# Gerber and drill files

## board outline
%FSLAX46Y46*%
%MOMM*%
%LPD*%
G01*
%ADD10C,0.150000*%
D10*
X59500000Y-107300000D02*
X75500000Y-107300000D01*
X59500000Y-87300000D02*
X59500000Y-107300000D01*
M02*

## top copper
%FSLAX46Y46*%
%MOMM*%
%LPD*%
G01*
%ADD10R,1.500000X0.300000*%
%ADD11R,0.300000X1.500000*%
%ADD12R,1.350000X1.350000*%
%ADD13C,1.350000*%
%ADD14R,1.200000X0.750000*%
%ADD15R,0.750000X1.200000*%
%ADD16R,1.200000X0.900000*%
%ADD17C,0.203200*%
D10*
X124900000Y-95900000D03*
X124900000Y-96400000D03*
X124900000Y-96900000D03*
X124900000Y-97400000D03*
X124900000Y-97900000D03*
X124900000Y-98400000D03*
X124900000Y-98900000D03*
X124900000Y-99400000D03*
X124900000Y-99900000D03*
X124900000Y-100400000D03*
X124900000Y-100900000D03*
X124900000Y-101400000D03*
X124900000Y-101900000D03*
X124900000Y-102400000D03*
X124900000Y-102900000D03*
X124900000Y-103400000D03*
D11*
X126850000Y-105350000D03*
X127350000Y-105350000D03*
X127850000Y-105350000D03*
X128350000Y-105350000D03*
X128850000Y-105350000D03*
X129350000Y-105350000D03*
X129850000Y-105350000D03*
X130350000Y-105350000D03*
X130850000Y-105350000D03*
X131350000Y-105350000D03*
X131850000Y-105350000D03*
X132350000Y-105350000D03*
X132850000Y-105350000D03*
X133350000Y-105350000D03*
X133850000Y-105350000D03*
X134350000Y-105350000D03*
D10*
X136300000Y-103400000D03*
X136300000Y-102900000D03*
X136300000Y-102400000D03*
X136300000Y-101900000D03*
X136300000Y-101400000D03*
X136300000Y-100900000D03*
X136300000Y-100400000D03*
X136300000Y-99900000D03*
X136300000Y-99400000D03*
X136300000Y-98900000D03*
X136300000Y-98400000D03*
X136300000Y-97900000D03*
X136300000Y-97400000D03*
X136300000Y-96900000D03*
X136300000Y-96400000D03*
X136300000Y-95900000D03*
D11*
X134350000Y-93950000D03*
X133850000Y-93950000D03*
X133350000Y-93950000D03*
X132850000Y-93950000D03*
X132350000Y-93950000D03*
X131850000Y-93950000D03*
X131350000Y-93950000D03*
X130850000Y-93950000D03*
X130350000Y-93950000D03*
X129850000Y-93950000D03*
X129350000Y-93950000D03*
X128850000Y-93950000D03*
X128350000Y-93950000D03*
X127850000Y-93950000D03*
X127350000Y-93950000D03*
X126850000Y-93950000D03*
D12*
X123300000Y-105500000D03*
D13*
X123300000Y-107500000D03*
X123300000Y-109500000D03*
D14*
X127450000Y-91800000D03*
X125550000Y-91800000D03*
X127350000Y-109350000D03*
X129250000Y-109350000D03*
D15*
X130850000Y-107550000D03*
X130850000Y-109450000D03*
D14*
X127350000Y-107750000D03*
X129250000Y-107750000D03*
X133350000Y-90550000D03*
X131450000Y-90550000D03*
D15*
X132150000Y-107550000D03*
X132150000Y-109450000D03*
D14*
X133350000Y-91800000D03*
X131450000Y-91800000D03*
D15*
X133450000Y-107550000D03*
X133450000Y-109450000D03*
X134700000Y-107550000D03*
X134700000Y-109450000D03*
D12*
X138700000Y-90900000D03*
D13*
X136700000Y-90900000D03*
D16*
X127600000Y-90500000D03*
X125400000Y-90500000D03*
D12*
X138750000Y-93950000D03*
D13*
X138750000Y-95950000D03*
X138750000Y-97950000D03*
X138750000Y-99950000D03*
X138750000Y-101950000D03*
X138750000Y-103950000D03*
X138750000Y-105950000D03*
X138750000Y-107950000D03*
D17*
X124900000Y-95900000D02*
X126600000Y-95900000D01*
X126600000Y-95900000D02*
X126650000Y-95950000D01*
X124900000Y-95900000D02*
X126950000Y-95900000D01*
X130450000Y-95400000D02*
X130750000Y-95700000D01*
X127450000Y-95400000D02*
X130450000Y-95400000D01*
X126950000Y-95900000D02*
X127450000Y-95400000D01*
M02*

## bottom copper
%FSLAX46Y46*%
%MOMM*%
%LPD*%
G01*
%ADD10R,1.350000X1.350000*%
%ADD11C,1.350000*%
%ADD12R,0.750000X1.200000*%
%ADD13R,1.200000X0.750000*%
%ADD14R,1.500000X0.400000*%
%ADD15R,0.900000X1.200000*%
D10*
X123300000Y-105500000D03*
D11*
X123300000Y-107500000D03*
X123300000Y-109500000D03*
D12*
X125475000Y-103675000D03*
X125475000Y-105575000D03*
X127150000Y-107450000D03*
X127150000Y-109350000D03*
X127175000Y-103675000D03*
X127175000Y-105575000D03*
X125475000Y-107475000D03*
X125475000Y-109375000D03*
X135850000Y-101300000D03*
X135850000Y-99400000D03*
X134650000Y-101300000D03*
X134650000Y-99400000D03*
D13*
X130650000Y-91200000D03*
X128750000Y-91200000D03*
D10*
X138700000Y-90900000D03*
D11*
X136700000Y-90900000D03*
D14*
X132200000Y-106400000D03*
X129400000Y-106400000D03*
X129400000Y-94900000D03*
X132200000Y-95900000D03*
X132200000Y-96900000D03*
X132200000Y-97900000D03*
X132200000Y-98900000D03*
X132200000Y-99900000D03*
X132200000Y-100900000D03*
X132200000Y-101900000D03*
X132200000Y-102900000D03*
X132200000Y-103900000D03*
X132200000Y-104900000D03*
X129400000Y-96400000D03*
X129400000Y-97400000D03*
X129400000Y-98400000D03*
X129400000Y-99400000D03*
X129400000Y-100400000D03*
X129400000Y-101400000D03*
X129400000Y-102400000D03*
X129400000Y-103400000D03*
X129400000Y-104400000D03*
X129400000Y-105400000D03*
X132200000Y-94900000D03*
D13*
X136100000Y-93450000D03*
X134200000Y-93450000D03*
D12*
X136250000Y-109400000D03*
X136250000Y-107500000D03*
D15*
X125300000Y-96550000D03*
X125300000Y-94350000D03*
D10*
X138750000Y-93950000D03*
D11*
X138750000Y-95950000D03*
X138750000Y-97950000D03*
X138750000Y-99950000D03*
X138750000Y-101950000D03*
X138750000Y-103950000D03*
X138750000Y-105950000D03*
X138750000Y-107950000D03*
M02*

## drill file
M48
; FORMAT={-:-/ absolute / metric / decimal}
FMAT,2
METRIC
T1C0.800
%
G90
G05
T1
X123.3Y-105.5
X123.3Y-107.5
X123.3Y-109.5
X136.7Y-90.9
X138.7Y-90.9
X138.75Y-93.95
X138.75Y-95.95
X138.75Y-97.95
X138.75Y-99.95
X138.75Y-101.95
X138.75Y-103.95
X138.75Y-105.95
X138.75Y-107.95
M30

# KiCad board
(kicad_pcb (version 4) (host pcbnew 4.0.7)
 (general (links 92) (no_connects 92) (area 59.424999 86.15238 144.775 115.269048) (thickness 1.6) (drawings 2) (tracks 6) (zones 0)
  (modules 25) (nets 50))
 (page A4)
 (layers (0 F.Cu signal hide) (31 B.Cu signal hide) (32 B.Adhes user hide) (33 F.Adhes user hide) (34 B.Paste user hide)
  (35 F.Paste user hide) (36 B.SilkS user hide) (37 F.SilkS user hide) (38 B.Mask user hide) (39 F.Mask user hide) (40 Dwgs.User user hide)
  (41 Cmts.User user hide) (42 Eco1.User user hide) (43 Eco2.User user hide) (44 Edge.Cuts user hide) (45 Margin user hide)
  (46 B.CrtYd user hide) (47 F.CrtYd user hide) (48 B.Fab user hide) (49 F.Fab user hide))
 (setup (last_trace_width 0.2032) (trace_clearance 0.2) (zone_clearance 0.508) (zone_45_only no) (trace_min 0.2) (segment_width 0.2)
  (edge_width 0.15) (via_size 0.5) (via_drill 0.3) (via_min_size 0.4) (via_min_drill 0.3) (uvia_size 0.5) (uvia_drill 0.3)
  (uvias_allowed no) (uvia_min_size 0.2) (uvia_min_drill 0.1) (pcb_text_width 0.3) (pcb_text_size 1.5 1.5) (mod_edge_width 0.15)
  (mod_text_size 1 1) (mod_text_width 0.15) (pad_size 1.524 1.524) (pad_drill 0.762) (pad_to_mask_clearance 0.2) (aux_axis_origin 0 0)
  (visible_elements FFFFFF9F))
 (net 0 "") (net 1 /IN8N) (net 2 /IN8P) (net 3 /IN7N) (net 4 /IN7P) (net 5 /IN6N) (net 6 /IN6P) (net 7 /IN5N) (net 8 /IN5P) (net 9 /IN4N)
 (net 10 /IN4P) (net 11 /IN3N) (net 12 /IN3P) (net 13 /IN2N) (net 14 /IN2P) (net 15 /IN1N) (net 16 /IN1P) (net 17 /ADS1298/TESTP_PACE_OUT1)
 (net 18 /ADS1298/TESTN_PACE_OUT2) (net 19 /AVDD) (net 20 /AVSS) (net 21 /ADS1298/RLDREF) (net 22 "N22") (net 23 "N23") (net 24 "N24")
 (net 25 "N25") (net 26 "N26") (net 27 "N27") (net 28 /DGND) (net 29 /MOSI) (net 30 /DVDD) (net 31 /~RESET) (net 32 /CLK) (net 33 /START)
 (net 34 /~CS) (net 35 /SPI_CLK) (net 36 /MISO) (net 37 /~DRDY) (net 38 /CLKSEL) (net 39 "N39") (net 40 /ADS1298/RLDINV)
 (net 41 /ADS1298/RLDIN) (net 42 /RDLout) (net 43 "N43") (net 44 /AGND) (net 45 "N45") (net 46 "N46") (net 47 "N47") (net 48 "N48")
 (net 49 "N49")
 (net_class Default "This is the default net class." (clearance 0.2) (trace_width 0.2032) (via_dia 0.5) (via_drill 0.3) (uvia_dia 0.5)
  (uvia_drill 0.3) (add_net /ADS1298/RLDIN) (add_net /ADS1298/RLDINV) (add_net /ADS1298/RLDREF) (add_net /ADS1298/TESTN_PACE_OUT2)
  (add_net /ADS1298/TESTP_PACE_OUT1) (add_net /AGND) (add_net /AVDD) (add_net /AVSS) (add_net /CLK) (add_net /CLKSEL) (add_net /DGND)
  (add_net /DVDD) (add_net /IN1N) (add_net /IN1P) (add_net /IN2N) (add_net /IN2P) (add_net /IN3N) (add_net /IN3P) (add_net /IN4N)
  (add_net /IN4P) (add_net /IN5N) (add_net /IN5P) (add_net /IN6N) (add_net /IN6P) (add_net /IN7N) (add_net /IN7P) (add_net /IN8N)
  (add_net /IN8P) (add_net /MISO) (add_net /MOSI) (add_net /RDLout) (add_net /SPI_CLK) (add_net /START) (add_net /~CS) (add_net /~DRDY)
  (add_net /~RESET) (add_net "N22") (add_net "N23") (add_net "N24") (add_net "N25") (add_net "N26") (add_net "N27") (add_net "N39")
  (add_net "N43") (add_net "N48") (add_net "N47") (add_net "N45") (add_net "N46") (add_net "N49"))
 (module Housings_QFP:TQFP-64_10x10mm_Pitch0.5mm (layer F.Cu) (at 130.6 99.65)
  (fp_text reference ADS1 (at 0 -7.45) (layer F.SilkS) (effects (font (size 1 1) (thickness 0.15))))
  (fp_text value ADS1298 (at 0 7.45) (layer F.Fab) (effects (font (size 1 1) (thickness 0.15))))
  (pad 1 smd rect (at -5.7 -3.75) (size 1.5 0.3) (layers F.Cu F.Paste F.Mask) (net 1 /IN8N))
  (pad 2 smd rect (at -5.7 -3.25) (size 1.5 0.3) (layers F.Cu F.Paste F.Mask) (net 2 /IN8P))
  (pad 3 smd rect (at -5.7 -2.75) (size 1.5 0.3) (layers F.Cu F.Paste F.Mask) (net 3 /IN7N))
  (pad 4 smd rect (at -5.7 -2.25) (size 1.5 0.3) (layers F.Cu F.Paste F.Mask) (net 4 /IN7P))
  (pad 5 smd rect (at -5.7 -1.75) (size 1.5 0.3) (layers F.Cu F.Paste F.Mask) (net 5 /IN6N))
  (pad 6 smd rect (at -5.7 -1.25) (size 1.5 0.3) (layers F.Cu F.Paste F.Mask) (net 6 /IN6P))
  (pad 7 smd rect (at -5.7 -0.75) (size 1.5 0.3) (layers F.Cu F.Paste F.Mask) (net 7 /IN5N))
  (pad 8 smd rect (at -5.7 -0.25) (size 1.5 0.3) (layers F.Cu F.Paste F.Mask) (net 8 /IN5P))
  (pad 9 smd rect (at -5.7 0.25) (size 1.5 0.3) (layers F.Cu F.Paste F.Mask) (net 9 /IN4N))
  (pad 10 smd rect (at -5.7 0.75) (size 1.5 0.3) (layers F.Cu F.Paste F.Mask) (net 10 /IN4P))
  (pad 11 smd rect (at -5.7 1.25) (size 1.5 0.3) (layers F.Cu F.Paste F.Mask) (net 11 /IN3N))
  (pad 12 smd rect (at -5.7 1.75) (size 1.5 0.3) (layers F.Cu F.Paste F.Mask) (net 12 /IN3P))
  (pad 13 smd rect (at -5.7 2.25) (size 1.5 0.3) (layers F.Cu F.Paste F.Mask) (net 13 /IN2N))
  (pad 14 smd rect (at -5.7 2.75) (size 1.5 0.3) (layers F.Cu F.Paste F.Mask) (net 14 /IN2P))
  (pad 15 smd rect (at -5.7 3.25) (size 1.5 0.3) (layers F.Cu F.Paste F.Mask) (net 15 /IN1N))
  (pad 16 smd rect (at -5.7 3.75) (size 1.5 0.3) (layers F.Cu F.Paste F.Mask) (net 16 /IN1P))
  (pad 17 smd rect (at -3.75 5.7 90) (size 1.5 0.3) (layers F.Cu F.Paste F.Mask) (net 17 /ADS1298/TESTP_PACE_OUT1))
  (pad 18 smd rect (at -3.25 5.7 90) (size 1.5 0.3) (layers F.Cu F.Paste F.Mask) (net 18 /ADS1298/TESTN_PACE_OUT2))
  (pad 19 smd rect (at -2.75 5.7 90) (size 1.5 0.3) (layers F.Cu F.Paste F.Mask) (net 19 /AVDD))
  (pad 20 smd rect (at -2.25 5.7 90) (size 1.5 0.3) (layers F.Cu F.Paste F.Mask) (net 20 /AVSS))
  (pad 21 smd rect (at -1.75 5.7 90) (size 1.5 0.3) (layers F.Cu F.Paste F.Mask) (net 19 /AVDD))
  (pad 22 smd rect (at -1.25 5.7 90) (size 1.5 0.3) (layers F.Cu F.Paste F.Mask) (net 19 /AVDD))
  (pad 23 smd rect (at -0.75 5.7 90) (size 1.5 0.3) (layers F.Cu F.Paste F.Mask) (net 20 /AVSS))
  (pad 24 smd rect (at -0.25 5.7 90) (size 1.5 0.3) (layers F.Cu F.Paste F.Mask) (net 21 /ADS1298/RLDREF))
  (pad 25 smd rect (at 0.25 5.7 90) (size 1.5 0.3) (layers F.Cu F.Paste F.Mask) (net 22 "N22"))
  (pad 26 smd rect (at 0.75 5.7 90) (size 1.5 0.3) (layers F.Cu F.Paste F.Mask) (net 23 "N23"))
  (pad 27 smd rect (at 1.25 5.7 90) (size 1.5 0.3) (layers F.Cu F.Paste F.Mask) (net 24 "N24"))
  (pad 28 smd rect (at 1.75 5.7 90) (size 1.5 0.3) (layers F.Cu F.Paste F.Mask) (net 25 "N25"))
  (pad 29 smd rect (at 2.25 5.7 90) (size 1.5 0.3) (layers F.Cu F.Paste F.Mask) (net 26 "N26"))
  (pad 30 smd rect (at 2.75 5.7 90) (size 1.5 0.3) (layers F.Cu F.Paste F.Mask) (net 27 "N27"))
  (pad 31 smd rect (at 3.25 5.7 90) (size 1.5 0.3) (layers F.Cu F.Paste F.Mask) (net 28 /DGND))
  (pad 32 smd rect (at 3.75 5.7 90) (size 1.5 0.3) (layers F.Cu F.Paste F.Mask) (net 20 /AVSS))
  (pad 33 smd rect (at 5.7 3.75) (size 1.5 0.3) (layers F.Cu F.Paste F.Mask) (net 28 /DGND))
  (pad 34 smd rect (at 5.7 3.25) (size 1.5 0.3) (layers F.Cu F.Paste F.Mask) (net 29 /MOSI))
  (pad 35 smd rect (at 5.7 2.75) (size 1.5 0.3) (layers F.Cu F.Paste F.Mask) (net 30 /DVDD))
  (pad 36 smd rect (at 5.7 2.25) (size 1.5 0.3) (layers F.Cu F.Paste F.Mask) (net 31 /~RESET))
  (pad 37 smd rect (at 5.7 1.75) (size 1.5 0.3) (layers F.Cu F.Paste F.Mask) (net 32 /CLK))
  (pad 38 smd rect (at 5.7 1.25) (size 1.5 0.3) (layers F.Cu F.Paste F.Mask) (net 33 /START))
  (pad 39 smd rect (at 5.7 0.75) (size 1.5 0.3) (layers F.Cu F.Paste F.Mask) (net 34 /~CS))
  (pad 40 smd rect (at 5.7 0.25) (size 1.5 0.3) (layers F.Cu F.Paste F.Mask) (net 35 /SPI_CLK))
  (pad 41 smd rect (at 5.7 -0.25) (size 1.5 0.3) (layers F.Cu F.Paste F.Mask) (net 28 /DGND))
  (pad 42 smd rect (at 5.7 -0.75) (size 1.5 0.3) (layers F.Cu F.Paste F.Mask) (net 28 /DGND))
  (pad 43 smd rect (at 5.7 -1.25) (size 1.5 0.3) (layers F.Cu F.Paste F.Mask) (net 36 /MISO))
  (pad 44 smd rect (at 5.7 -1.75) (size 1.5 0.3) (layers F.Cu F.Paste F.Mask) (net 28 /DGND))
  (pad 45 smd rect (at 5.7 -2.25) (size 1.5 0.3) (layers F.Cu F.Paste F.Mask) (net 28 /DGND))
  (pad 46 smd rect (at 5.7 -2.75) (size 1.5 0.3) (layers F.Cu F.Paste F.Mask) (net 28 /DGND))
  (pad 47 smd rect (at 5.7 -3.25) (size 1.5 0.3) (layers F.Cu F.Paste F.Mask) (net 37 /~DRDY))
  (pad 48 smd rect (at 5.7 -3.75) (size 1.5 0.3) (layers F.Cu F.Paste F.Mask) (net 30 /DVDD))
  (pad 49 smd rect (at 3.75 -5.7 90) (size 1.5 0.3) (layers F.Cu F.Paste F.Mask) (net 28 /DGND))
  (pad 50 smd rect (at 3.25 -5.7 90) (size 1.5 0.3) (layers F.Cu F.Paste F.Mask) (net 30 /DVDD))
  (pad 51 smd rect (at 2.75 -5.7 90) (size 1.5 0.3) (layers F.Cu F.Paste F.Mask) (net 28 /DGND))
  (pad 52 smd rect (at 2.25 -5.7 90) (size 1.5 0.3) (layers F.Cu F.Paste F.Mask) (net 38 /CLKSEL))
  (pad 53 smd rect (at 1.75 -5.7 90) (size 1.5 0.3) (layers F.Cu F.Paste F.Mask) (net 20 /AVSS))
  (pad 54 smd rect (at 1.25 -5.7 90) (size 1.5 0.3) (layers F.Cu F.Paste F.Mask) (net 19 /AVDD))
  (pad 55 smd rect (at 0.75 -5.7 90) (size 1.5 0.3) (layers F.Cu F.Paste F.Mask) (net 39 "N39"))
  (pad 56 smd rect (at 0.25 -5.7 90) (size 1.5 0.3) (layers F.Cu F.Paste F.Mask) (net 19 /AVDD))
  (pad 57 smd rect (at -0.25 -5.7 90) (size 1.5 0.3) (layers F.Cu F.Paste F.Mask) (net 20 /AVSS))
  (pad 58 smd rect (at -0.75 -5.7 90) (size 1.5 0.3) (layers F.Cu F.Paste F.Mask) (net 20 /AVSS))
  (pad 59 smd rect (at -1.25 -5.7 90) (size 1.5 0.3) (layers F.Cu F.Paste F.Mask) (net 19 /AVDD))
  (pad 60 smd rect (at -1.75 -5.7 90) (size 1.5 0.3) (layers F.Cu F.Paste F.Mask) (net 21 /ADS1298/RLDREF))
  (pad 61 smd rect (at -2.25 -5.7 90) (size 1.5 0.3) (layers F.Cu F.Paste F.Mask) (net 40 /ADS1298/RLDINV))
  (pad 62 smd rect (at -2.75 -5.7 90) (size 1.5 0.3) (layers F.Cu F.Paste F.Mask) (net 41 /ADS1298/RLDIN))
  (pad 63 smd rect (at -3.25 -5.7 90) (size 1.5 0.3) (layers F.Cu F.Paste F.Mask) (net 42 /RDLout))
  (pad 64 smd rect (at -3.75 -5.7 90) (size 1.5 0.3) (layers F.Cu F.Paste F.Mask) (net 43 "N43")))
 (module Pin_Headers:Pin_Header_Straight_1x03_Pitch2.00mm (layer F.Cu) (at 123.3 105.5)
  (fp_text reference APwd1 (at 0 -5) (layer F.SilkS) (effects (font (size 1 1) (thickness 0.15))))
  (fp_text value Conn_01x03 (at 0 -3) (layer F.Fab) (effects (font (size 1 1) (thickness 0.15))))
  (pad 1 thru_hole rect (at 0 0) (size 1.35 1.35) (drill 0.8) (layers *.Cu *.Mask) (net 19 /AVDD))
  (pad 2 thru_hole circle (at 0 2) (size 1.35 1.35) (drill 0.8) (layers *.Cu *.Mask) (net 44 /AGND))
  (pad 3 thru_hole circle (at 0 4) (size 1.35 1.35) (drill 0.8) (layers *.Cu *.Mask) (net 20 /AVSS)))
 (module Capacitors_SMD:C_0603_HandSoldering (layer F.Cu) (at 126.5 91.8 180)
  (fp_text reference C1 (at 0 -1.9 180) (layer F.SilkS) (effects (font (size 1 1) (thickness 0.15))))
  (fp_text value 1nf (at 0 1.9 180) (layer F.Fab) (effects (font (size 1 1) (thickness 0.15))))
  (pad 1 smd rect (at -0.95 0 180) (size 1.2 0.75) (layers F.Cu F.Paste F.Mask) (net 40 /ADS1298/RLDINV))
  (pad 2 smd rect (at 0.95 0 180) (size 1.2 0.75) (layers F.Cu F.Paste F.Mask) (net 42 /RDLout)))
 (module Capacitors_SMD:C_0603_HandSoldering (layer B.Cu) (at 125.475 104.625 270)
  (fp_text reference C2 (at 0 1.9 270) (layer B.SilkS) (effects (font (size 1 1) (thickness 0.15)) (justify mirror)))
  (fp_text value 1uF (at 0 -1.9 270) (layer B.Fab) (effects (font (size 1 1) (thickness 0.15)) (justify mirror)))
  (pad 1 smd rect (at -0.95 0 270) (size 1.2 0.75) (layers B.Cu B.Paste B.Mask) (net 19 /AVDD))
  (pad 2 smd rect (at 0.95 0 270) (size 1.2 0.75) (layers B.Cu B.Paste B.Mask) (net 44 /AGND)))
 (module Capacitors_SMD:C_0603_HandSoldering (layer B.Cu) (at 127.15 108.4 270)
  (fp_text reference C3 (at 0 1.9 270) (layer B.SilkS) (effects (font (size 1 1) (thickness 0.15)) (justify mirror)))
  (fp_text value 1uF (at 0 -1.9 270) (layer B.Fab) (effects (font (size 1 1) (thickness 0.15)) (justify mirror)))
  (pad 1 smd rect (at -0.95 0 270) (size 1.2 0.75) (layers B.Cu B.Paste B.Mask) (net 44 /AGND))
  (pad 2 smd rect (at 0.95 0 270) (size 1.2 0.75) (layers B.Cu B.Paste B.Mask) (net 20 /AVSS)))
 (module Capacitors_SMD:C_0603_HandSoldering (layer B.Cu) (at 127.175 104.625 270)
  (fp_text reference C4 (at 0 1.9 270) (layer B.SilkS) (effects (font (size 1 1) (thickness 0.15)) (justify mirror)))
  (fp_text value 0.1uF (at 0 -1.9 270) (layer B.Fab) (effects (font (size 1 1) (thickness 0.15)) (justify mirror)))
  (pad 1 smd rect (at -0.95 0 270) (size 1.2 0.75) (layers B.Cu B.Paste B.Mask) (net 19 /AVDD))
  (pad 2 smd rect (at 0.95 0 270) (size 1.2 0.75) (layers B.Cu B.Paste B.Mask) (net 44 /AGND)))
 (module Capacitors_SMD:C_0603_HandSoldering (layer B.Cu) (at 125.475 108.425 270)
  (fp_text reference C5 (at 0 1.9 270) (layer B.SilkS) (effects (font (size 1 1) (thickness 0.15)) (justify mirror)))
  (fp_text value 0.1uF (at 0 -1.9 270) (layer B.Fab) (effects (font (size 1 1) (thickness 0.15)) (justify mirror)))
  (pad 1 smd rect (at -0.95 0 270) (size 1.2 0.75) (layers B.Cu B.Paste B.Mask) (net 44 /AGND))
  (pad 2 smd rect (at 0.95 0 270) (size 1.2 0.75) (layers B.Cu B.Paste B.Mask) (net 20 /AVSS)))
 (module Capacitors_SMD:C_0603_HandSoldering (layer B.Cu) (at 135.85 100.35 90)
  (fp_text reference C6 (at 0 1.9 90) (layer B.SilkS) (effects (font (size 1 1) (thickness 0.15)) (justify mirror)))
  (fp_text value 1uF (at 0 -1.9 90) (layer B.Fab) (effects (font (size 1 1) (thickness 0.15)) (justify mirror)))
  (pad 1 smd rect (at -0.95 0 90) (size 1.2 0.75) (layers B.Cu B.Paste B.Mask) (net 30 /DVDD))
  (pad 2 smd rect (at 0.95 0 90) (size 1.2 0.75) (layers B.Cu B.Paste B.Mask) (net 28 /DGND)))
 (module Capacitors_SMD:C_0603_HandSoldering (layer B.Cu) (at 134.65 100.35 90)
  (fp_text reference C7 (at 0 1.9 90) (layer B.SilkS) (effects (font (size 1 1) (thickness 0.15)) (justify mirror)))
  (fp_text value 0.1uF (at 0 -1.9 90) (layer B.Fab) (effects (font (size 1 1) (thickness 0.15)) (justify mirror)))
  (pad 1 smd rect (at -0.95 0 90) (size 1.2 0.75) (layers B.Cu B.Paste B.Mask) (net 30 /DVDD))
  (pad 2 smd rect (at 0.95 0 90) (size 1.2 0.75) (layers B.Cu B.Paste B.Mask) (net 28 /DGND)))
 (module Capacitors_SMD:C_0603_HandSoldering (layer B.Cu) (at 129.7 91.2 180)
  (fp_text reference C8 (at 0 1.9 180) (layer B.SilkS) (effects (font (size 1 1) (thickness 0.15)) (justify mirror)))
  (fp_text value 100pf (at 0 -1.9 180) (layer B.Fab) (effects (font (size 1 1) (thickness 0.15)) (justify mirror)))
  (pad 1 smd rect (at -0.95 0 180) (size 1.2 0.75) (layers B.Cu B.Paste B.Mask) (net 20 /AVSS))
  (pad 2 smd rect (at 0.95 0 180) (size 1.2 0.75) (layers B.Cu B.Paste B.Mask) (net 43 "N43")))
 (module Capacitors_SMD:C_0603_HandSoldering (layer F.Cu) (at 128.3 109.35)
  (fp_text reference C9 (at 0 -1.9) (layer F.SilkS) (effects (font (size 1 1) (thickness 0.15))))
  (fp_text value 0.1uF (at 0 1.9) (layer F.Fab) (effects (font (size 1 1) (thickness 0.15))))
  (pad 1 smd rect (at -0.95 0) (size 1.2 0.75) (layers F.Cu F.Paste F.Mask) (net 21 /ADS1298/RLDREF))
  (pad 2 smd rect (at 0.95 0) (size 1.2 0.75) (layers F.Cu F.Paste F.Mask) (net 22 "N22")))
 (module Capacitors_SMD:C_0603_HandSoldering (layer F.Cu) (at 130.85 108.5 270)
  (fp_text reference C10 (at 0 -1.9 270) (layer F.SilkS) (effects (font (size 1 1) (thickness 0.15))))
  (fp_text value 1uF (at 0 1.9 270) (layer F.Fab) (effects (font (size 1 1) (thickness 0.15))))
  (pad 1 smd rect (at -0.95 0 270) (size 1.2 0.75) (layers F.Cu F.Paste F.Mask) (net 22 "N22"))
  (pad 2 smd rect (at 0.95 0 270) (size 1.2 0.75) (layers F.Cu F.Paste F.Mask) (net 20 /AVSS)))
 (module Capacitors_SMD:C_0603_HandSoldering (layer F.Cu) (at 128.3 107.75)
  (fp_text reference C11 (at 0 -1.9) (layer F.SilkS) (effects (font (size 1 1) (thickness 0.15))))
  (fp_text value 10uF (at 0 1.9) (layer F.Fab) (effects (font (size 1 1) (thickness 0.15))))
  (pad 1 smd rect (at -0.95 0) (size 1.2 0.75) (layers F.Cu F.Paste F.Mask) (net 21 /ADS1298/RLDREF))
  (pad 2 smd rect (at 0.95 0) (size 1.2 0.75) (layers F.Cu F.Paste F.Mask) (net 22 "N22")))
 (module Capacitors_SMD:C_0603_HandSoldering (layer F.Cu) (at 132.4 90.55 180)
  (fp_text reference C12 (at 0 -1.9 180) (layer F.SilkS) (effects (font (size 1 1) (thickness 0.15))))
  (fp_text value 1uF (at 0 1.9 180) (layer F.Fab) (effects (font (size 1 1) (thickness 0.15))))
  (pad 1 smd rect (at -0.95 0 180) (size 1.2 0.75) (layers F.Cu F.Paste F.Mask) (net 20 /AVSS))
  (pad 2 smd rect (at 0.95 0 180) (size 1.2 0.75) (layers F.Cu F.Paste F.Mask) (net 39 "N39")))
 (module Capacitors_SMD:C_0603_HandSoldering (layer F.Cu) (at 132.15 108.5 270)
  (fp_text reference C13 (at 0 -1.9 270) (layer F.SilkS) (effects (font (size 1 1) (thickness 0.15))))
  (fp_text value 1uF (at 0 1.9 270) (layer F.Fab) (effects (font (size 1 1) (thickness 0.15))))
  (pad 1 smd rect (at -0.95 0 270) (size 1.2 0.75) (layers F.Cu F.Paste F.Mask) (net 23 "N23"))
  (pad 2 smd rect (at 0.95 0 270) (size 1.2 0.75) (layers F.Cu F.Paste F.Mask) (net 20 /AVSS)))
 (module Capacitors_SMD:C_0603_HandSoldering (layer F.Cu) (at 132.4 91.8 180)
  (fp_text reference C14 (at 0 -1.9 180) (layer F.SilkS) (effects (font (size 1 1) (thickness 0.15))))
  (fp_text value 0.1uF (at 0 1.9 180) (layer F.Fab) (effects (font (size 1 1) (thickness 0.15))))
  (pad 1 smd rect (at -0.95 0 180) (size 1.2 0.75) (layers F.Cu F.Paste F.Mask) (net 20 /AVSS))
  (pad 2 smd rect (at 0.95 0 180) (size 1.2 0.75) (layers F.Cu F.Paste F.Mask) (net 39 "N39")))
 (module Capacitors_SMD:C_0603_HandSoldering (layer F.Cu) (at 133.45 108.5 270)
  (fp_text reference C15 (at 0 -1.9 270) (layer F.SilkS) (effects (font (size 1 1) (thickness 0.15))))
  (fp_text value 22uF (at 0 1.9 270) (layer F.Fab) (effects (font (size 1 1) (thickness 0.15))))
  (pad 1 smd rect (at -0.95 0 270) (size 1.2 0.75) (layers F.Cu F.Paste F.Mask) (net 25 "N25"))
  (pad 2 smd rect (at 0.95 0 270) (size 1.2 0.75) (layers F.Cu F.Paste F.Mask) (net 20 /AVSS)))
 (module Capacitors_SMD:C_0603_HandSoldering (layer F.Cu) (at 134.7 108.5 270)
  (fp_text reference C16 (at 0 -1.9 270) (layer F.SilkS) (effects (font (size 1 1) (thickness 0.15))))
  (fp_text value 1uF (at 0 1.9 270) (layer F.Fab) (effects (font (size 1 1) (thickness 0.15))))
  (pad 1 smd rect (at -0.95 0 270) (size 1.2 0.75) (layers F.Cu F.Paste F.Mask) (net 27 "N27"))
  (pad 2 smd rect (at 0.95 0 270) (size 1.2 0.75) (layers F.Cu F.Paste F.Mask) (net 20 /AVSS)))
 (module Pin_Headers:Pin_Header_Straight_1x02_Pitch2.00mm (layer F.Cu) (at 138.7 90.9 270)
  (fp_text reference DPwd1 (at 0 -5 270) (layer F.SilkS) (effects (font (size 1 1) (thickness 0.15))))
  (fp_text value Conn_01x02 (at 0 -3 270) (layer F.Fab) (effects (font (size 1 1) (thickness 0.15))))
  (pad 1 thru_hole rect (at 0 0 270) (size 1.35 1.35) (drill 0.8) (layers *.Cu *.Mask) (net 30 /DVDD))
  (pad 2 thru_hole circle (at 0 2 270) (size 1.35 1.35) (drill 0.8) (layers *.Cu *.Mask) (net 28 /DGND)))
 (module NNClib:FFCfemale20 (layer B.Cu) (at 132.95 95.9 270)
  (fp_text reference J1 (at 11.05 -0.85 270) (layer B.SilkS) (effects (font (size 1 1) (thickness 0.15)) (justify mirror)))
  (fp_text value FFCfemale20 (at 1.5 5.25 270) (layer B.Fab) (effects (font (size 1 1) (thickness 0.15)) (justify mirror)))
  (pad 42 smd rect (at 10.5 0.75 270) (size 0.4 1.5) (layers B.Cu B.Paste B.Mask) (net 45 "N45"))
  (pad 43 smd rect (at 10.5 3.55 270) (size 0.4 1.5) (layers B.Cu B.Paste B.Mask) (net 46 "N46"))
  (pad 41 smd rect (at -1 3.55 270) (size 0.4 1.5) (layers B.Cu B.Paste B.Mask) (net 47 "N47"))
  (pad 1 smd rect (at 0 0.75 90) (size 0.4 1.5) (layers B.Cu B.Paste B.Mask) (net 44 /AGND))
  (pad 3 smd rect (at 1 0.75 90) (size 0.4 1.5) (layers B.Cu B.Paste B.Mask) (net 1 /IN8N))
  (pad 5 smd rect (at 2 0.75 90) (size 0.4 1.5) (layers B.Cu B.Paste B.Mask) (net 3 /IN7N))
  (pad 7 smd rect (at 3 0.75 90) (size 0.4 1.5) (layers B.Cu B.Paste B.Mask) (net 5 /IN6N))
  (pad 9 smd rect (at 4 0.75 90) (size 0.4 1.5) (layers B.Cu B.Paste B.Mask) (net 7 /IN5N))
  (pad 11 smd rect (at 5 0.75 90) (size 0.4 1.5) (layers B.Cu B.Paste B.Mask) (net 9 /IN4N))
  (pad 13 smd rect (at 6 0.75 90) (size 0.4 1.5) (layers B.Cu B.Paste B.Mask) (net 11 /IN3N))
  (pad 15 smd rect (at 7 0.75 90) (size 0.4 1.5) (layers B.Cu B.Paste B.Mask) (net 13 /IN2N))
  (pad 17 smd rect (at 8 0.75 90) (size 0.4 1.5) (layers B.Cu B.Paste B.Mask) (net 15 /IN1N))
  (pad 19 smd rect (at 9 0.75 90) (size 0.4 1.5) (layers B.Cu B.Paste B.Mask) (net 42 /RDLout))
  (pad 2 smd rect (at 0.5 3.55 90) (size 0.4 1.5) (layers B.Cu B.Paste B.Mask) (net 42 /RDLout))
  (pad 4 smd rect (at 1.5 3.55 90) (size 0.4 1.5) (layers B.Cu B.Paste B.Mask) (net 2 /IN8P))
  (pad 6 smd rect (at 2.5 3.55 90) (size 0.4 1.5) (layers B.Cu B.Paste B.Mask) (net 4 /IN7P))
  (pad 8 smd rect (at 3.5 3.55 90) (size 0.4 1.5) (layers B.Cu B.Paste B.Mask) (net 6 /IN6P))
  (pad 10 smd rect (at 4.5 3.55 90) (size 0.4 1.5) (layers B.Cu B.Paste B.Mask) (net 8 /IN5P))
  (pad 12 smd rect (at 5.5 3.55 90) (size 0.4 1.5) (layers B.Cu B.Paste B.Mask) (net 10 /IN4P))
  (pad 14 smd rect (at 6.5 3.55 90) (size 0.4 1.5) (layers B.Cu B.Paste B.Mask) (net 12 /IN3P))
  (pad 16 smd rect (at 7.5 3.55 90) (size 0.4 1.5) (layers B.Cu B.Paste B.Mask) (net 14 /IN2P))
  (pad 18 smd rect (at 8.5 3.55 90) (size 0.4 1.5) (layers B.Cu B.Paste B.Mask) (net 16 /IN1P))
  (pad 20 smd rect (at 9.5 3.55 90) (size 0.4 1.5) (layers B.Cu B.Paste B.Mask) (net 44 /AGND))
  (pad 40 smd rect (at -1 0.75 270) (size 0.4 1.5) (layers B.Cu B.Paste B.Mask) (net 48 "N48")))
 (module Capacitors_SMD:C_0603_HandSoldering (layer B.Cu) (at 135.15 93.45 180)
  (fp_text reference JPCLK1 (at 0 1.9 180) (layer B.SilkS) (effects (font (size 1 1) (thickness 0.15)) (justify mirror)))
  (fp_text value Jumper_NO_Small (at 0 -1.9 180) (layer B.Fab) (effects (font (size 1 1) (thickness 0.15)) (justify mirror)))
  (pad 1 smd rect (at -0.95 0 180) (size 1.2 0.75) (layers B.Cu B.Paste B.Mask) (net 30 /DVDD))
  (pad 2 smd rect (at 0.95 0 180) (size 1.2 0.75) (layers B.Cu B.Paste B.Mask) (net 38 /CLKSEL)))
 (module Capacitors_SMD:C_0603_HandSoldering (layer B.Cu) (at 136.25 108.45 90)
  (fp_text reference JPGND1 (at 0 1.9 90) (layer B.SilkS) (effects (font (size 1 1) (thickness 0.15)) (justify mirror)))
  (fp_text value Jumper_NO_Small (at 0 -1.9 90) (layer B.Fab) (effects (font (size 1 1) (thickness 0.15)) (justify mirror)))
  (pad 1 smd rect (at -0.95 0 90) (size 1.2 0.75) (layers B.Cu B.Paste B.Mask) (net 44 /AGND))
  (pad 2 smd rect (at 0.95 0 90) (size 1.2 0.75) (layers B.Cu B.Paste B.Mask) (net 28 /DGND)))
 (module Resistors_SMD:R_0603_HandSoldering (layer F.Cu) (at 126.5 90.5 180)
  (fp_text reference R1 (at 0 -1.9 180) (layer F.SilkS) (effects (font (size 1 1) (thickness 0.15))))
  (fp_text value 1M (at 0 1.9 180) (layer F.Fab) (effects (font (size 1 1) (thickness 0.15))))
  (pad 1 smd rect (at -1.1 0 180) (size 1.2 0.9) (layers F.Cu F.Paste F.Mask) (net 40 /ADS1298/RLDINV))
  (pad 2 smd rect (at 1.1 0 180) (size 1.2 0.9) (layers F.Cu F.Paste F.Mask) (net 42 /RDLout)))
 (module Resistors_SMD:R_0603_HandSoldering (layer B.Cu) (at 125.3 95.45 90)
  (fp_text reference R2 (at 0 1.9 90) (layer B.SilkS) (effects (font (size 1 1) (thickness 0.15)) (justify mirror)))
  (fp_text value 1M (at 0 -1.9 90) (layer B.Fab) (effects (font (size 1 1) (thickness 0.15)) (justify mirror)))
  (pad 1 smd rect (at -1.1 0 90) (size 1.2 0.9) (layers B.Cu B.Paste B.Mask) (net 44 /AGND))
  (pad 2 smd rect (at 1.1 0 90) (size 1.2 0.9) (layers B.Cu B.Paste B.Mask) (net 41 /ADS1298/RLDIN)))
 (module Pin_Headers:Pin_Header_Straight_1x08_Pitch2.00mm (layer F.Cu) (at 138.75 93.95)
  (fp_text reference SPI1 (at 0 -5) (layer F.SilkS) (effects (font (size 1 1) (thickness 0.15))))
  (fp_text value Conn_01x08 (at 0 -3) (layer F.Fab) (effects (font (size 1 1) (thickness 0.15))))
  (pad 1 thru_hole rect (at 0 0) (size 1.35 1.35) (drill 0.8) (layers *.Cu *.Mask) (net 37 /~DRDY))
  (pad 2 thru_hole circle (at 0 2) (size 1.35 1.35) (drill 0.8) (layers *.Cu *.Mask) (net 36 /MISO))
  (pad 3 thru_hole circle (at 0 4) (size 1.35 1.35) (drill 0.8) (layers *.Cu *.Mask) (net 35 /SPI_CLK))
  (pad 4 thru_hole circle (at 0 6) (size 1.35 1.35) (drill 0.8) (layers *.Cu *.Mask) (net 34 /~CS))
  (pad 5 thru_hole circle (at 0 8) (size 1.35 1.35) (drill 0.8) (layers *.Cu *.Mask) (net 33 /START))
  (pad 6 thru_hole circle (at 0 10) (size 1.35 1.35) (drill 0.8) (layers *.Cu *.Mask) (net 31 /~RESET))
  (pad 7 thru_hole circle (at 0 12) (size 1.35 1.35) (drill 0.8) (layers *.Cu *.Mask) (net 29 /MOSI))
  (pad 8 thru_hole circle (at 0 14) (size 1.35 1.35) (drill 0.8) (layers *.Cu *.Mask) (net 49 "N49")))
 (gr_line (start 59.5 107.3) (end 75.5 107.3) (angle 90) (layer Edge.Cuts) (width 0.15))
 (gr_line (start 59.5 87.3) (end 59.5 107.3) (angle 90) (layer Edge.Cuts) (width 0.15))
 (segment (start 124.9 95.9) (end 126.6 95.9) (width 0.2032) (layer F.Cu) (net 1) (status 400000))
 (segment (start 126.6 95.9) (end 126.65 95.95) (width 0.2032) (layer F.Cu) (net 1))
 (segment (start 124.9 95.9) (end 126.95 95.9) (width 0.2032) (layer F.Cu) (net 1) (status 400000))
 (segment (start 130.45 95.4) (end 130.75 95.7) (width 0.2032) (layer F.Cu) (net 1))
 (segment (start 127.45 95.4) (end 130.45 95.4) (width 0.2032) (layer F.Cu) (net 1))
 (segment (start 126.95 95.9) (end 127.45 95.4) (width 0.2032) (layer F.Cu) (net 1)))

